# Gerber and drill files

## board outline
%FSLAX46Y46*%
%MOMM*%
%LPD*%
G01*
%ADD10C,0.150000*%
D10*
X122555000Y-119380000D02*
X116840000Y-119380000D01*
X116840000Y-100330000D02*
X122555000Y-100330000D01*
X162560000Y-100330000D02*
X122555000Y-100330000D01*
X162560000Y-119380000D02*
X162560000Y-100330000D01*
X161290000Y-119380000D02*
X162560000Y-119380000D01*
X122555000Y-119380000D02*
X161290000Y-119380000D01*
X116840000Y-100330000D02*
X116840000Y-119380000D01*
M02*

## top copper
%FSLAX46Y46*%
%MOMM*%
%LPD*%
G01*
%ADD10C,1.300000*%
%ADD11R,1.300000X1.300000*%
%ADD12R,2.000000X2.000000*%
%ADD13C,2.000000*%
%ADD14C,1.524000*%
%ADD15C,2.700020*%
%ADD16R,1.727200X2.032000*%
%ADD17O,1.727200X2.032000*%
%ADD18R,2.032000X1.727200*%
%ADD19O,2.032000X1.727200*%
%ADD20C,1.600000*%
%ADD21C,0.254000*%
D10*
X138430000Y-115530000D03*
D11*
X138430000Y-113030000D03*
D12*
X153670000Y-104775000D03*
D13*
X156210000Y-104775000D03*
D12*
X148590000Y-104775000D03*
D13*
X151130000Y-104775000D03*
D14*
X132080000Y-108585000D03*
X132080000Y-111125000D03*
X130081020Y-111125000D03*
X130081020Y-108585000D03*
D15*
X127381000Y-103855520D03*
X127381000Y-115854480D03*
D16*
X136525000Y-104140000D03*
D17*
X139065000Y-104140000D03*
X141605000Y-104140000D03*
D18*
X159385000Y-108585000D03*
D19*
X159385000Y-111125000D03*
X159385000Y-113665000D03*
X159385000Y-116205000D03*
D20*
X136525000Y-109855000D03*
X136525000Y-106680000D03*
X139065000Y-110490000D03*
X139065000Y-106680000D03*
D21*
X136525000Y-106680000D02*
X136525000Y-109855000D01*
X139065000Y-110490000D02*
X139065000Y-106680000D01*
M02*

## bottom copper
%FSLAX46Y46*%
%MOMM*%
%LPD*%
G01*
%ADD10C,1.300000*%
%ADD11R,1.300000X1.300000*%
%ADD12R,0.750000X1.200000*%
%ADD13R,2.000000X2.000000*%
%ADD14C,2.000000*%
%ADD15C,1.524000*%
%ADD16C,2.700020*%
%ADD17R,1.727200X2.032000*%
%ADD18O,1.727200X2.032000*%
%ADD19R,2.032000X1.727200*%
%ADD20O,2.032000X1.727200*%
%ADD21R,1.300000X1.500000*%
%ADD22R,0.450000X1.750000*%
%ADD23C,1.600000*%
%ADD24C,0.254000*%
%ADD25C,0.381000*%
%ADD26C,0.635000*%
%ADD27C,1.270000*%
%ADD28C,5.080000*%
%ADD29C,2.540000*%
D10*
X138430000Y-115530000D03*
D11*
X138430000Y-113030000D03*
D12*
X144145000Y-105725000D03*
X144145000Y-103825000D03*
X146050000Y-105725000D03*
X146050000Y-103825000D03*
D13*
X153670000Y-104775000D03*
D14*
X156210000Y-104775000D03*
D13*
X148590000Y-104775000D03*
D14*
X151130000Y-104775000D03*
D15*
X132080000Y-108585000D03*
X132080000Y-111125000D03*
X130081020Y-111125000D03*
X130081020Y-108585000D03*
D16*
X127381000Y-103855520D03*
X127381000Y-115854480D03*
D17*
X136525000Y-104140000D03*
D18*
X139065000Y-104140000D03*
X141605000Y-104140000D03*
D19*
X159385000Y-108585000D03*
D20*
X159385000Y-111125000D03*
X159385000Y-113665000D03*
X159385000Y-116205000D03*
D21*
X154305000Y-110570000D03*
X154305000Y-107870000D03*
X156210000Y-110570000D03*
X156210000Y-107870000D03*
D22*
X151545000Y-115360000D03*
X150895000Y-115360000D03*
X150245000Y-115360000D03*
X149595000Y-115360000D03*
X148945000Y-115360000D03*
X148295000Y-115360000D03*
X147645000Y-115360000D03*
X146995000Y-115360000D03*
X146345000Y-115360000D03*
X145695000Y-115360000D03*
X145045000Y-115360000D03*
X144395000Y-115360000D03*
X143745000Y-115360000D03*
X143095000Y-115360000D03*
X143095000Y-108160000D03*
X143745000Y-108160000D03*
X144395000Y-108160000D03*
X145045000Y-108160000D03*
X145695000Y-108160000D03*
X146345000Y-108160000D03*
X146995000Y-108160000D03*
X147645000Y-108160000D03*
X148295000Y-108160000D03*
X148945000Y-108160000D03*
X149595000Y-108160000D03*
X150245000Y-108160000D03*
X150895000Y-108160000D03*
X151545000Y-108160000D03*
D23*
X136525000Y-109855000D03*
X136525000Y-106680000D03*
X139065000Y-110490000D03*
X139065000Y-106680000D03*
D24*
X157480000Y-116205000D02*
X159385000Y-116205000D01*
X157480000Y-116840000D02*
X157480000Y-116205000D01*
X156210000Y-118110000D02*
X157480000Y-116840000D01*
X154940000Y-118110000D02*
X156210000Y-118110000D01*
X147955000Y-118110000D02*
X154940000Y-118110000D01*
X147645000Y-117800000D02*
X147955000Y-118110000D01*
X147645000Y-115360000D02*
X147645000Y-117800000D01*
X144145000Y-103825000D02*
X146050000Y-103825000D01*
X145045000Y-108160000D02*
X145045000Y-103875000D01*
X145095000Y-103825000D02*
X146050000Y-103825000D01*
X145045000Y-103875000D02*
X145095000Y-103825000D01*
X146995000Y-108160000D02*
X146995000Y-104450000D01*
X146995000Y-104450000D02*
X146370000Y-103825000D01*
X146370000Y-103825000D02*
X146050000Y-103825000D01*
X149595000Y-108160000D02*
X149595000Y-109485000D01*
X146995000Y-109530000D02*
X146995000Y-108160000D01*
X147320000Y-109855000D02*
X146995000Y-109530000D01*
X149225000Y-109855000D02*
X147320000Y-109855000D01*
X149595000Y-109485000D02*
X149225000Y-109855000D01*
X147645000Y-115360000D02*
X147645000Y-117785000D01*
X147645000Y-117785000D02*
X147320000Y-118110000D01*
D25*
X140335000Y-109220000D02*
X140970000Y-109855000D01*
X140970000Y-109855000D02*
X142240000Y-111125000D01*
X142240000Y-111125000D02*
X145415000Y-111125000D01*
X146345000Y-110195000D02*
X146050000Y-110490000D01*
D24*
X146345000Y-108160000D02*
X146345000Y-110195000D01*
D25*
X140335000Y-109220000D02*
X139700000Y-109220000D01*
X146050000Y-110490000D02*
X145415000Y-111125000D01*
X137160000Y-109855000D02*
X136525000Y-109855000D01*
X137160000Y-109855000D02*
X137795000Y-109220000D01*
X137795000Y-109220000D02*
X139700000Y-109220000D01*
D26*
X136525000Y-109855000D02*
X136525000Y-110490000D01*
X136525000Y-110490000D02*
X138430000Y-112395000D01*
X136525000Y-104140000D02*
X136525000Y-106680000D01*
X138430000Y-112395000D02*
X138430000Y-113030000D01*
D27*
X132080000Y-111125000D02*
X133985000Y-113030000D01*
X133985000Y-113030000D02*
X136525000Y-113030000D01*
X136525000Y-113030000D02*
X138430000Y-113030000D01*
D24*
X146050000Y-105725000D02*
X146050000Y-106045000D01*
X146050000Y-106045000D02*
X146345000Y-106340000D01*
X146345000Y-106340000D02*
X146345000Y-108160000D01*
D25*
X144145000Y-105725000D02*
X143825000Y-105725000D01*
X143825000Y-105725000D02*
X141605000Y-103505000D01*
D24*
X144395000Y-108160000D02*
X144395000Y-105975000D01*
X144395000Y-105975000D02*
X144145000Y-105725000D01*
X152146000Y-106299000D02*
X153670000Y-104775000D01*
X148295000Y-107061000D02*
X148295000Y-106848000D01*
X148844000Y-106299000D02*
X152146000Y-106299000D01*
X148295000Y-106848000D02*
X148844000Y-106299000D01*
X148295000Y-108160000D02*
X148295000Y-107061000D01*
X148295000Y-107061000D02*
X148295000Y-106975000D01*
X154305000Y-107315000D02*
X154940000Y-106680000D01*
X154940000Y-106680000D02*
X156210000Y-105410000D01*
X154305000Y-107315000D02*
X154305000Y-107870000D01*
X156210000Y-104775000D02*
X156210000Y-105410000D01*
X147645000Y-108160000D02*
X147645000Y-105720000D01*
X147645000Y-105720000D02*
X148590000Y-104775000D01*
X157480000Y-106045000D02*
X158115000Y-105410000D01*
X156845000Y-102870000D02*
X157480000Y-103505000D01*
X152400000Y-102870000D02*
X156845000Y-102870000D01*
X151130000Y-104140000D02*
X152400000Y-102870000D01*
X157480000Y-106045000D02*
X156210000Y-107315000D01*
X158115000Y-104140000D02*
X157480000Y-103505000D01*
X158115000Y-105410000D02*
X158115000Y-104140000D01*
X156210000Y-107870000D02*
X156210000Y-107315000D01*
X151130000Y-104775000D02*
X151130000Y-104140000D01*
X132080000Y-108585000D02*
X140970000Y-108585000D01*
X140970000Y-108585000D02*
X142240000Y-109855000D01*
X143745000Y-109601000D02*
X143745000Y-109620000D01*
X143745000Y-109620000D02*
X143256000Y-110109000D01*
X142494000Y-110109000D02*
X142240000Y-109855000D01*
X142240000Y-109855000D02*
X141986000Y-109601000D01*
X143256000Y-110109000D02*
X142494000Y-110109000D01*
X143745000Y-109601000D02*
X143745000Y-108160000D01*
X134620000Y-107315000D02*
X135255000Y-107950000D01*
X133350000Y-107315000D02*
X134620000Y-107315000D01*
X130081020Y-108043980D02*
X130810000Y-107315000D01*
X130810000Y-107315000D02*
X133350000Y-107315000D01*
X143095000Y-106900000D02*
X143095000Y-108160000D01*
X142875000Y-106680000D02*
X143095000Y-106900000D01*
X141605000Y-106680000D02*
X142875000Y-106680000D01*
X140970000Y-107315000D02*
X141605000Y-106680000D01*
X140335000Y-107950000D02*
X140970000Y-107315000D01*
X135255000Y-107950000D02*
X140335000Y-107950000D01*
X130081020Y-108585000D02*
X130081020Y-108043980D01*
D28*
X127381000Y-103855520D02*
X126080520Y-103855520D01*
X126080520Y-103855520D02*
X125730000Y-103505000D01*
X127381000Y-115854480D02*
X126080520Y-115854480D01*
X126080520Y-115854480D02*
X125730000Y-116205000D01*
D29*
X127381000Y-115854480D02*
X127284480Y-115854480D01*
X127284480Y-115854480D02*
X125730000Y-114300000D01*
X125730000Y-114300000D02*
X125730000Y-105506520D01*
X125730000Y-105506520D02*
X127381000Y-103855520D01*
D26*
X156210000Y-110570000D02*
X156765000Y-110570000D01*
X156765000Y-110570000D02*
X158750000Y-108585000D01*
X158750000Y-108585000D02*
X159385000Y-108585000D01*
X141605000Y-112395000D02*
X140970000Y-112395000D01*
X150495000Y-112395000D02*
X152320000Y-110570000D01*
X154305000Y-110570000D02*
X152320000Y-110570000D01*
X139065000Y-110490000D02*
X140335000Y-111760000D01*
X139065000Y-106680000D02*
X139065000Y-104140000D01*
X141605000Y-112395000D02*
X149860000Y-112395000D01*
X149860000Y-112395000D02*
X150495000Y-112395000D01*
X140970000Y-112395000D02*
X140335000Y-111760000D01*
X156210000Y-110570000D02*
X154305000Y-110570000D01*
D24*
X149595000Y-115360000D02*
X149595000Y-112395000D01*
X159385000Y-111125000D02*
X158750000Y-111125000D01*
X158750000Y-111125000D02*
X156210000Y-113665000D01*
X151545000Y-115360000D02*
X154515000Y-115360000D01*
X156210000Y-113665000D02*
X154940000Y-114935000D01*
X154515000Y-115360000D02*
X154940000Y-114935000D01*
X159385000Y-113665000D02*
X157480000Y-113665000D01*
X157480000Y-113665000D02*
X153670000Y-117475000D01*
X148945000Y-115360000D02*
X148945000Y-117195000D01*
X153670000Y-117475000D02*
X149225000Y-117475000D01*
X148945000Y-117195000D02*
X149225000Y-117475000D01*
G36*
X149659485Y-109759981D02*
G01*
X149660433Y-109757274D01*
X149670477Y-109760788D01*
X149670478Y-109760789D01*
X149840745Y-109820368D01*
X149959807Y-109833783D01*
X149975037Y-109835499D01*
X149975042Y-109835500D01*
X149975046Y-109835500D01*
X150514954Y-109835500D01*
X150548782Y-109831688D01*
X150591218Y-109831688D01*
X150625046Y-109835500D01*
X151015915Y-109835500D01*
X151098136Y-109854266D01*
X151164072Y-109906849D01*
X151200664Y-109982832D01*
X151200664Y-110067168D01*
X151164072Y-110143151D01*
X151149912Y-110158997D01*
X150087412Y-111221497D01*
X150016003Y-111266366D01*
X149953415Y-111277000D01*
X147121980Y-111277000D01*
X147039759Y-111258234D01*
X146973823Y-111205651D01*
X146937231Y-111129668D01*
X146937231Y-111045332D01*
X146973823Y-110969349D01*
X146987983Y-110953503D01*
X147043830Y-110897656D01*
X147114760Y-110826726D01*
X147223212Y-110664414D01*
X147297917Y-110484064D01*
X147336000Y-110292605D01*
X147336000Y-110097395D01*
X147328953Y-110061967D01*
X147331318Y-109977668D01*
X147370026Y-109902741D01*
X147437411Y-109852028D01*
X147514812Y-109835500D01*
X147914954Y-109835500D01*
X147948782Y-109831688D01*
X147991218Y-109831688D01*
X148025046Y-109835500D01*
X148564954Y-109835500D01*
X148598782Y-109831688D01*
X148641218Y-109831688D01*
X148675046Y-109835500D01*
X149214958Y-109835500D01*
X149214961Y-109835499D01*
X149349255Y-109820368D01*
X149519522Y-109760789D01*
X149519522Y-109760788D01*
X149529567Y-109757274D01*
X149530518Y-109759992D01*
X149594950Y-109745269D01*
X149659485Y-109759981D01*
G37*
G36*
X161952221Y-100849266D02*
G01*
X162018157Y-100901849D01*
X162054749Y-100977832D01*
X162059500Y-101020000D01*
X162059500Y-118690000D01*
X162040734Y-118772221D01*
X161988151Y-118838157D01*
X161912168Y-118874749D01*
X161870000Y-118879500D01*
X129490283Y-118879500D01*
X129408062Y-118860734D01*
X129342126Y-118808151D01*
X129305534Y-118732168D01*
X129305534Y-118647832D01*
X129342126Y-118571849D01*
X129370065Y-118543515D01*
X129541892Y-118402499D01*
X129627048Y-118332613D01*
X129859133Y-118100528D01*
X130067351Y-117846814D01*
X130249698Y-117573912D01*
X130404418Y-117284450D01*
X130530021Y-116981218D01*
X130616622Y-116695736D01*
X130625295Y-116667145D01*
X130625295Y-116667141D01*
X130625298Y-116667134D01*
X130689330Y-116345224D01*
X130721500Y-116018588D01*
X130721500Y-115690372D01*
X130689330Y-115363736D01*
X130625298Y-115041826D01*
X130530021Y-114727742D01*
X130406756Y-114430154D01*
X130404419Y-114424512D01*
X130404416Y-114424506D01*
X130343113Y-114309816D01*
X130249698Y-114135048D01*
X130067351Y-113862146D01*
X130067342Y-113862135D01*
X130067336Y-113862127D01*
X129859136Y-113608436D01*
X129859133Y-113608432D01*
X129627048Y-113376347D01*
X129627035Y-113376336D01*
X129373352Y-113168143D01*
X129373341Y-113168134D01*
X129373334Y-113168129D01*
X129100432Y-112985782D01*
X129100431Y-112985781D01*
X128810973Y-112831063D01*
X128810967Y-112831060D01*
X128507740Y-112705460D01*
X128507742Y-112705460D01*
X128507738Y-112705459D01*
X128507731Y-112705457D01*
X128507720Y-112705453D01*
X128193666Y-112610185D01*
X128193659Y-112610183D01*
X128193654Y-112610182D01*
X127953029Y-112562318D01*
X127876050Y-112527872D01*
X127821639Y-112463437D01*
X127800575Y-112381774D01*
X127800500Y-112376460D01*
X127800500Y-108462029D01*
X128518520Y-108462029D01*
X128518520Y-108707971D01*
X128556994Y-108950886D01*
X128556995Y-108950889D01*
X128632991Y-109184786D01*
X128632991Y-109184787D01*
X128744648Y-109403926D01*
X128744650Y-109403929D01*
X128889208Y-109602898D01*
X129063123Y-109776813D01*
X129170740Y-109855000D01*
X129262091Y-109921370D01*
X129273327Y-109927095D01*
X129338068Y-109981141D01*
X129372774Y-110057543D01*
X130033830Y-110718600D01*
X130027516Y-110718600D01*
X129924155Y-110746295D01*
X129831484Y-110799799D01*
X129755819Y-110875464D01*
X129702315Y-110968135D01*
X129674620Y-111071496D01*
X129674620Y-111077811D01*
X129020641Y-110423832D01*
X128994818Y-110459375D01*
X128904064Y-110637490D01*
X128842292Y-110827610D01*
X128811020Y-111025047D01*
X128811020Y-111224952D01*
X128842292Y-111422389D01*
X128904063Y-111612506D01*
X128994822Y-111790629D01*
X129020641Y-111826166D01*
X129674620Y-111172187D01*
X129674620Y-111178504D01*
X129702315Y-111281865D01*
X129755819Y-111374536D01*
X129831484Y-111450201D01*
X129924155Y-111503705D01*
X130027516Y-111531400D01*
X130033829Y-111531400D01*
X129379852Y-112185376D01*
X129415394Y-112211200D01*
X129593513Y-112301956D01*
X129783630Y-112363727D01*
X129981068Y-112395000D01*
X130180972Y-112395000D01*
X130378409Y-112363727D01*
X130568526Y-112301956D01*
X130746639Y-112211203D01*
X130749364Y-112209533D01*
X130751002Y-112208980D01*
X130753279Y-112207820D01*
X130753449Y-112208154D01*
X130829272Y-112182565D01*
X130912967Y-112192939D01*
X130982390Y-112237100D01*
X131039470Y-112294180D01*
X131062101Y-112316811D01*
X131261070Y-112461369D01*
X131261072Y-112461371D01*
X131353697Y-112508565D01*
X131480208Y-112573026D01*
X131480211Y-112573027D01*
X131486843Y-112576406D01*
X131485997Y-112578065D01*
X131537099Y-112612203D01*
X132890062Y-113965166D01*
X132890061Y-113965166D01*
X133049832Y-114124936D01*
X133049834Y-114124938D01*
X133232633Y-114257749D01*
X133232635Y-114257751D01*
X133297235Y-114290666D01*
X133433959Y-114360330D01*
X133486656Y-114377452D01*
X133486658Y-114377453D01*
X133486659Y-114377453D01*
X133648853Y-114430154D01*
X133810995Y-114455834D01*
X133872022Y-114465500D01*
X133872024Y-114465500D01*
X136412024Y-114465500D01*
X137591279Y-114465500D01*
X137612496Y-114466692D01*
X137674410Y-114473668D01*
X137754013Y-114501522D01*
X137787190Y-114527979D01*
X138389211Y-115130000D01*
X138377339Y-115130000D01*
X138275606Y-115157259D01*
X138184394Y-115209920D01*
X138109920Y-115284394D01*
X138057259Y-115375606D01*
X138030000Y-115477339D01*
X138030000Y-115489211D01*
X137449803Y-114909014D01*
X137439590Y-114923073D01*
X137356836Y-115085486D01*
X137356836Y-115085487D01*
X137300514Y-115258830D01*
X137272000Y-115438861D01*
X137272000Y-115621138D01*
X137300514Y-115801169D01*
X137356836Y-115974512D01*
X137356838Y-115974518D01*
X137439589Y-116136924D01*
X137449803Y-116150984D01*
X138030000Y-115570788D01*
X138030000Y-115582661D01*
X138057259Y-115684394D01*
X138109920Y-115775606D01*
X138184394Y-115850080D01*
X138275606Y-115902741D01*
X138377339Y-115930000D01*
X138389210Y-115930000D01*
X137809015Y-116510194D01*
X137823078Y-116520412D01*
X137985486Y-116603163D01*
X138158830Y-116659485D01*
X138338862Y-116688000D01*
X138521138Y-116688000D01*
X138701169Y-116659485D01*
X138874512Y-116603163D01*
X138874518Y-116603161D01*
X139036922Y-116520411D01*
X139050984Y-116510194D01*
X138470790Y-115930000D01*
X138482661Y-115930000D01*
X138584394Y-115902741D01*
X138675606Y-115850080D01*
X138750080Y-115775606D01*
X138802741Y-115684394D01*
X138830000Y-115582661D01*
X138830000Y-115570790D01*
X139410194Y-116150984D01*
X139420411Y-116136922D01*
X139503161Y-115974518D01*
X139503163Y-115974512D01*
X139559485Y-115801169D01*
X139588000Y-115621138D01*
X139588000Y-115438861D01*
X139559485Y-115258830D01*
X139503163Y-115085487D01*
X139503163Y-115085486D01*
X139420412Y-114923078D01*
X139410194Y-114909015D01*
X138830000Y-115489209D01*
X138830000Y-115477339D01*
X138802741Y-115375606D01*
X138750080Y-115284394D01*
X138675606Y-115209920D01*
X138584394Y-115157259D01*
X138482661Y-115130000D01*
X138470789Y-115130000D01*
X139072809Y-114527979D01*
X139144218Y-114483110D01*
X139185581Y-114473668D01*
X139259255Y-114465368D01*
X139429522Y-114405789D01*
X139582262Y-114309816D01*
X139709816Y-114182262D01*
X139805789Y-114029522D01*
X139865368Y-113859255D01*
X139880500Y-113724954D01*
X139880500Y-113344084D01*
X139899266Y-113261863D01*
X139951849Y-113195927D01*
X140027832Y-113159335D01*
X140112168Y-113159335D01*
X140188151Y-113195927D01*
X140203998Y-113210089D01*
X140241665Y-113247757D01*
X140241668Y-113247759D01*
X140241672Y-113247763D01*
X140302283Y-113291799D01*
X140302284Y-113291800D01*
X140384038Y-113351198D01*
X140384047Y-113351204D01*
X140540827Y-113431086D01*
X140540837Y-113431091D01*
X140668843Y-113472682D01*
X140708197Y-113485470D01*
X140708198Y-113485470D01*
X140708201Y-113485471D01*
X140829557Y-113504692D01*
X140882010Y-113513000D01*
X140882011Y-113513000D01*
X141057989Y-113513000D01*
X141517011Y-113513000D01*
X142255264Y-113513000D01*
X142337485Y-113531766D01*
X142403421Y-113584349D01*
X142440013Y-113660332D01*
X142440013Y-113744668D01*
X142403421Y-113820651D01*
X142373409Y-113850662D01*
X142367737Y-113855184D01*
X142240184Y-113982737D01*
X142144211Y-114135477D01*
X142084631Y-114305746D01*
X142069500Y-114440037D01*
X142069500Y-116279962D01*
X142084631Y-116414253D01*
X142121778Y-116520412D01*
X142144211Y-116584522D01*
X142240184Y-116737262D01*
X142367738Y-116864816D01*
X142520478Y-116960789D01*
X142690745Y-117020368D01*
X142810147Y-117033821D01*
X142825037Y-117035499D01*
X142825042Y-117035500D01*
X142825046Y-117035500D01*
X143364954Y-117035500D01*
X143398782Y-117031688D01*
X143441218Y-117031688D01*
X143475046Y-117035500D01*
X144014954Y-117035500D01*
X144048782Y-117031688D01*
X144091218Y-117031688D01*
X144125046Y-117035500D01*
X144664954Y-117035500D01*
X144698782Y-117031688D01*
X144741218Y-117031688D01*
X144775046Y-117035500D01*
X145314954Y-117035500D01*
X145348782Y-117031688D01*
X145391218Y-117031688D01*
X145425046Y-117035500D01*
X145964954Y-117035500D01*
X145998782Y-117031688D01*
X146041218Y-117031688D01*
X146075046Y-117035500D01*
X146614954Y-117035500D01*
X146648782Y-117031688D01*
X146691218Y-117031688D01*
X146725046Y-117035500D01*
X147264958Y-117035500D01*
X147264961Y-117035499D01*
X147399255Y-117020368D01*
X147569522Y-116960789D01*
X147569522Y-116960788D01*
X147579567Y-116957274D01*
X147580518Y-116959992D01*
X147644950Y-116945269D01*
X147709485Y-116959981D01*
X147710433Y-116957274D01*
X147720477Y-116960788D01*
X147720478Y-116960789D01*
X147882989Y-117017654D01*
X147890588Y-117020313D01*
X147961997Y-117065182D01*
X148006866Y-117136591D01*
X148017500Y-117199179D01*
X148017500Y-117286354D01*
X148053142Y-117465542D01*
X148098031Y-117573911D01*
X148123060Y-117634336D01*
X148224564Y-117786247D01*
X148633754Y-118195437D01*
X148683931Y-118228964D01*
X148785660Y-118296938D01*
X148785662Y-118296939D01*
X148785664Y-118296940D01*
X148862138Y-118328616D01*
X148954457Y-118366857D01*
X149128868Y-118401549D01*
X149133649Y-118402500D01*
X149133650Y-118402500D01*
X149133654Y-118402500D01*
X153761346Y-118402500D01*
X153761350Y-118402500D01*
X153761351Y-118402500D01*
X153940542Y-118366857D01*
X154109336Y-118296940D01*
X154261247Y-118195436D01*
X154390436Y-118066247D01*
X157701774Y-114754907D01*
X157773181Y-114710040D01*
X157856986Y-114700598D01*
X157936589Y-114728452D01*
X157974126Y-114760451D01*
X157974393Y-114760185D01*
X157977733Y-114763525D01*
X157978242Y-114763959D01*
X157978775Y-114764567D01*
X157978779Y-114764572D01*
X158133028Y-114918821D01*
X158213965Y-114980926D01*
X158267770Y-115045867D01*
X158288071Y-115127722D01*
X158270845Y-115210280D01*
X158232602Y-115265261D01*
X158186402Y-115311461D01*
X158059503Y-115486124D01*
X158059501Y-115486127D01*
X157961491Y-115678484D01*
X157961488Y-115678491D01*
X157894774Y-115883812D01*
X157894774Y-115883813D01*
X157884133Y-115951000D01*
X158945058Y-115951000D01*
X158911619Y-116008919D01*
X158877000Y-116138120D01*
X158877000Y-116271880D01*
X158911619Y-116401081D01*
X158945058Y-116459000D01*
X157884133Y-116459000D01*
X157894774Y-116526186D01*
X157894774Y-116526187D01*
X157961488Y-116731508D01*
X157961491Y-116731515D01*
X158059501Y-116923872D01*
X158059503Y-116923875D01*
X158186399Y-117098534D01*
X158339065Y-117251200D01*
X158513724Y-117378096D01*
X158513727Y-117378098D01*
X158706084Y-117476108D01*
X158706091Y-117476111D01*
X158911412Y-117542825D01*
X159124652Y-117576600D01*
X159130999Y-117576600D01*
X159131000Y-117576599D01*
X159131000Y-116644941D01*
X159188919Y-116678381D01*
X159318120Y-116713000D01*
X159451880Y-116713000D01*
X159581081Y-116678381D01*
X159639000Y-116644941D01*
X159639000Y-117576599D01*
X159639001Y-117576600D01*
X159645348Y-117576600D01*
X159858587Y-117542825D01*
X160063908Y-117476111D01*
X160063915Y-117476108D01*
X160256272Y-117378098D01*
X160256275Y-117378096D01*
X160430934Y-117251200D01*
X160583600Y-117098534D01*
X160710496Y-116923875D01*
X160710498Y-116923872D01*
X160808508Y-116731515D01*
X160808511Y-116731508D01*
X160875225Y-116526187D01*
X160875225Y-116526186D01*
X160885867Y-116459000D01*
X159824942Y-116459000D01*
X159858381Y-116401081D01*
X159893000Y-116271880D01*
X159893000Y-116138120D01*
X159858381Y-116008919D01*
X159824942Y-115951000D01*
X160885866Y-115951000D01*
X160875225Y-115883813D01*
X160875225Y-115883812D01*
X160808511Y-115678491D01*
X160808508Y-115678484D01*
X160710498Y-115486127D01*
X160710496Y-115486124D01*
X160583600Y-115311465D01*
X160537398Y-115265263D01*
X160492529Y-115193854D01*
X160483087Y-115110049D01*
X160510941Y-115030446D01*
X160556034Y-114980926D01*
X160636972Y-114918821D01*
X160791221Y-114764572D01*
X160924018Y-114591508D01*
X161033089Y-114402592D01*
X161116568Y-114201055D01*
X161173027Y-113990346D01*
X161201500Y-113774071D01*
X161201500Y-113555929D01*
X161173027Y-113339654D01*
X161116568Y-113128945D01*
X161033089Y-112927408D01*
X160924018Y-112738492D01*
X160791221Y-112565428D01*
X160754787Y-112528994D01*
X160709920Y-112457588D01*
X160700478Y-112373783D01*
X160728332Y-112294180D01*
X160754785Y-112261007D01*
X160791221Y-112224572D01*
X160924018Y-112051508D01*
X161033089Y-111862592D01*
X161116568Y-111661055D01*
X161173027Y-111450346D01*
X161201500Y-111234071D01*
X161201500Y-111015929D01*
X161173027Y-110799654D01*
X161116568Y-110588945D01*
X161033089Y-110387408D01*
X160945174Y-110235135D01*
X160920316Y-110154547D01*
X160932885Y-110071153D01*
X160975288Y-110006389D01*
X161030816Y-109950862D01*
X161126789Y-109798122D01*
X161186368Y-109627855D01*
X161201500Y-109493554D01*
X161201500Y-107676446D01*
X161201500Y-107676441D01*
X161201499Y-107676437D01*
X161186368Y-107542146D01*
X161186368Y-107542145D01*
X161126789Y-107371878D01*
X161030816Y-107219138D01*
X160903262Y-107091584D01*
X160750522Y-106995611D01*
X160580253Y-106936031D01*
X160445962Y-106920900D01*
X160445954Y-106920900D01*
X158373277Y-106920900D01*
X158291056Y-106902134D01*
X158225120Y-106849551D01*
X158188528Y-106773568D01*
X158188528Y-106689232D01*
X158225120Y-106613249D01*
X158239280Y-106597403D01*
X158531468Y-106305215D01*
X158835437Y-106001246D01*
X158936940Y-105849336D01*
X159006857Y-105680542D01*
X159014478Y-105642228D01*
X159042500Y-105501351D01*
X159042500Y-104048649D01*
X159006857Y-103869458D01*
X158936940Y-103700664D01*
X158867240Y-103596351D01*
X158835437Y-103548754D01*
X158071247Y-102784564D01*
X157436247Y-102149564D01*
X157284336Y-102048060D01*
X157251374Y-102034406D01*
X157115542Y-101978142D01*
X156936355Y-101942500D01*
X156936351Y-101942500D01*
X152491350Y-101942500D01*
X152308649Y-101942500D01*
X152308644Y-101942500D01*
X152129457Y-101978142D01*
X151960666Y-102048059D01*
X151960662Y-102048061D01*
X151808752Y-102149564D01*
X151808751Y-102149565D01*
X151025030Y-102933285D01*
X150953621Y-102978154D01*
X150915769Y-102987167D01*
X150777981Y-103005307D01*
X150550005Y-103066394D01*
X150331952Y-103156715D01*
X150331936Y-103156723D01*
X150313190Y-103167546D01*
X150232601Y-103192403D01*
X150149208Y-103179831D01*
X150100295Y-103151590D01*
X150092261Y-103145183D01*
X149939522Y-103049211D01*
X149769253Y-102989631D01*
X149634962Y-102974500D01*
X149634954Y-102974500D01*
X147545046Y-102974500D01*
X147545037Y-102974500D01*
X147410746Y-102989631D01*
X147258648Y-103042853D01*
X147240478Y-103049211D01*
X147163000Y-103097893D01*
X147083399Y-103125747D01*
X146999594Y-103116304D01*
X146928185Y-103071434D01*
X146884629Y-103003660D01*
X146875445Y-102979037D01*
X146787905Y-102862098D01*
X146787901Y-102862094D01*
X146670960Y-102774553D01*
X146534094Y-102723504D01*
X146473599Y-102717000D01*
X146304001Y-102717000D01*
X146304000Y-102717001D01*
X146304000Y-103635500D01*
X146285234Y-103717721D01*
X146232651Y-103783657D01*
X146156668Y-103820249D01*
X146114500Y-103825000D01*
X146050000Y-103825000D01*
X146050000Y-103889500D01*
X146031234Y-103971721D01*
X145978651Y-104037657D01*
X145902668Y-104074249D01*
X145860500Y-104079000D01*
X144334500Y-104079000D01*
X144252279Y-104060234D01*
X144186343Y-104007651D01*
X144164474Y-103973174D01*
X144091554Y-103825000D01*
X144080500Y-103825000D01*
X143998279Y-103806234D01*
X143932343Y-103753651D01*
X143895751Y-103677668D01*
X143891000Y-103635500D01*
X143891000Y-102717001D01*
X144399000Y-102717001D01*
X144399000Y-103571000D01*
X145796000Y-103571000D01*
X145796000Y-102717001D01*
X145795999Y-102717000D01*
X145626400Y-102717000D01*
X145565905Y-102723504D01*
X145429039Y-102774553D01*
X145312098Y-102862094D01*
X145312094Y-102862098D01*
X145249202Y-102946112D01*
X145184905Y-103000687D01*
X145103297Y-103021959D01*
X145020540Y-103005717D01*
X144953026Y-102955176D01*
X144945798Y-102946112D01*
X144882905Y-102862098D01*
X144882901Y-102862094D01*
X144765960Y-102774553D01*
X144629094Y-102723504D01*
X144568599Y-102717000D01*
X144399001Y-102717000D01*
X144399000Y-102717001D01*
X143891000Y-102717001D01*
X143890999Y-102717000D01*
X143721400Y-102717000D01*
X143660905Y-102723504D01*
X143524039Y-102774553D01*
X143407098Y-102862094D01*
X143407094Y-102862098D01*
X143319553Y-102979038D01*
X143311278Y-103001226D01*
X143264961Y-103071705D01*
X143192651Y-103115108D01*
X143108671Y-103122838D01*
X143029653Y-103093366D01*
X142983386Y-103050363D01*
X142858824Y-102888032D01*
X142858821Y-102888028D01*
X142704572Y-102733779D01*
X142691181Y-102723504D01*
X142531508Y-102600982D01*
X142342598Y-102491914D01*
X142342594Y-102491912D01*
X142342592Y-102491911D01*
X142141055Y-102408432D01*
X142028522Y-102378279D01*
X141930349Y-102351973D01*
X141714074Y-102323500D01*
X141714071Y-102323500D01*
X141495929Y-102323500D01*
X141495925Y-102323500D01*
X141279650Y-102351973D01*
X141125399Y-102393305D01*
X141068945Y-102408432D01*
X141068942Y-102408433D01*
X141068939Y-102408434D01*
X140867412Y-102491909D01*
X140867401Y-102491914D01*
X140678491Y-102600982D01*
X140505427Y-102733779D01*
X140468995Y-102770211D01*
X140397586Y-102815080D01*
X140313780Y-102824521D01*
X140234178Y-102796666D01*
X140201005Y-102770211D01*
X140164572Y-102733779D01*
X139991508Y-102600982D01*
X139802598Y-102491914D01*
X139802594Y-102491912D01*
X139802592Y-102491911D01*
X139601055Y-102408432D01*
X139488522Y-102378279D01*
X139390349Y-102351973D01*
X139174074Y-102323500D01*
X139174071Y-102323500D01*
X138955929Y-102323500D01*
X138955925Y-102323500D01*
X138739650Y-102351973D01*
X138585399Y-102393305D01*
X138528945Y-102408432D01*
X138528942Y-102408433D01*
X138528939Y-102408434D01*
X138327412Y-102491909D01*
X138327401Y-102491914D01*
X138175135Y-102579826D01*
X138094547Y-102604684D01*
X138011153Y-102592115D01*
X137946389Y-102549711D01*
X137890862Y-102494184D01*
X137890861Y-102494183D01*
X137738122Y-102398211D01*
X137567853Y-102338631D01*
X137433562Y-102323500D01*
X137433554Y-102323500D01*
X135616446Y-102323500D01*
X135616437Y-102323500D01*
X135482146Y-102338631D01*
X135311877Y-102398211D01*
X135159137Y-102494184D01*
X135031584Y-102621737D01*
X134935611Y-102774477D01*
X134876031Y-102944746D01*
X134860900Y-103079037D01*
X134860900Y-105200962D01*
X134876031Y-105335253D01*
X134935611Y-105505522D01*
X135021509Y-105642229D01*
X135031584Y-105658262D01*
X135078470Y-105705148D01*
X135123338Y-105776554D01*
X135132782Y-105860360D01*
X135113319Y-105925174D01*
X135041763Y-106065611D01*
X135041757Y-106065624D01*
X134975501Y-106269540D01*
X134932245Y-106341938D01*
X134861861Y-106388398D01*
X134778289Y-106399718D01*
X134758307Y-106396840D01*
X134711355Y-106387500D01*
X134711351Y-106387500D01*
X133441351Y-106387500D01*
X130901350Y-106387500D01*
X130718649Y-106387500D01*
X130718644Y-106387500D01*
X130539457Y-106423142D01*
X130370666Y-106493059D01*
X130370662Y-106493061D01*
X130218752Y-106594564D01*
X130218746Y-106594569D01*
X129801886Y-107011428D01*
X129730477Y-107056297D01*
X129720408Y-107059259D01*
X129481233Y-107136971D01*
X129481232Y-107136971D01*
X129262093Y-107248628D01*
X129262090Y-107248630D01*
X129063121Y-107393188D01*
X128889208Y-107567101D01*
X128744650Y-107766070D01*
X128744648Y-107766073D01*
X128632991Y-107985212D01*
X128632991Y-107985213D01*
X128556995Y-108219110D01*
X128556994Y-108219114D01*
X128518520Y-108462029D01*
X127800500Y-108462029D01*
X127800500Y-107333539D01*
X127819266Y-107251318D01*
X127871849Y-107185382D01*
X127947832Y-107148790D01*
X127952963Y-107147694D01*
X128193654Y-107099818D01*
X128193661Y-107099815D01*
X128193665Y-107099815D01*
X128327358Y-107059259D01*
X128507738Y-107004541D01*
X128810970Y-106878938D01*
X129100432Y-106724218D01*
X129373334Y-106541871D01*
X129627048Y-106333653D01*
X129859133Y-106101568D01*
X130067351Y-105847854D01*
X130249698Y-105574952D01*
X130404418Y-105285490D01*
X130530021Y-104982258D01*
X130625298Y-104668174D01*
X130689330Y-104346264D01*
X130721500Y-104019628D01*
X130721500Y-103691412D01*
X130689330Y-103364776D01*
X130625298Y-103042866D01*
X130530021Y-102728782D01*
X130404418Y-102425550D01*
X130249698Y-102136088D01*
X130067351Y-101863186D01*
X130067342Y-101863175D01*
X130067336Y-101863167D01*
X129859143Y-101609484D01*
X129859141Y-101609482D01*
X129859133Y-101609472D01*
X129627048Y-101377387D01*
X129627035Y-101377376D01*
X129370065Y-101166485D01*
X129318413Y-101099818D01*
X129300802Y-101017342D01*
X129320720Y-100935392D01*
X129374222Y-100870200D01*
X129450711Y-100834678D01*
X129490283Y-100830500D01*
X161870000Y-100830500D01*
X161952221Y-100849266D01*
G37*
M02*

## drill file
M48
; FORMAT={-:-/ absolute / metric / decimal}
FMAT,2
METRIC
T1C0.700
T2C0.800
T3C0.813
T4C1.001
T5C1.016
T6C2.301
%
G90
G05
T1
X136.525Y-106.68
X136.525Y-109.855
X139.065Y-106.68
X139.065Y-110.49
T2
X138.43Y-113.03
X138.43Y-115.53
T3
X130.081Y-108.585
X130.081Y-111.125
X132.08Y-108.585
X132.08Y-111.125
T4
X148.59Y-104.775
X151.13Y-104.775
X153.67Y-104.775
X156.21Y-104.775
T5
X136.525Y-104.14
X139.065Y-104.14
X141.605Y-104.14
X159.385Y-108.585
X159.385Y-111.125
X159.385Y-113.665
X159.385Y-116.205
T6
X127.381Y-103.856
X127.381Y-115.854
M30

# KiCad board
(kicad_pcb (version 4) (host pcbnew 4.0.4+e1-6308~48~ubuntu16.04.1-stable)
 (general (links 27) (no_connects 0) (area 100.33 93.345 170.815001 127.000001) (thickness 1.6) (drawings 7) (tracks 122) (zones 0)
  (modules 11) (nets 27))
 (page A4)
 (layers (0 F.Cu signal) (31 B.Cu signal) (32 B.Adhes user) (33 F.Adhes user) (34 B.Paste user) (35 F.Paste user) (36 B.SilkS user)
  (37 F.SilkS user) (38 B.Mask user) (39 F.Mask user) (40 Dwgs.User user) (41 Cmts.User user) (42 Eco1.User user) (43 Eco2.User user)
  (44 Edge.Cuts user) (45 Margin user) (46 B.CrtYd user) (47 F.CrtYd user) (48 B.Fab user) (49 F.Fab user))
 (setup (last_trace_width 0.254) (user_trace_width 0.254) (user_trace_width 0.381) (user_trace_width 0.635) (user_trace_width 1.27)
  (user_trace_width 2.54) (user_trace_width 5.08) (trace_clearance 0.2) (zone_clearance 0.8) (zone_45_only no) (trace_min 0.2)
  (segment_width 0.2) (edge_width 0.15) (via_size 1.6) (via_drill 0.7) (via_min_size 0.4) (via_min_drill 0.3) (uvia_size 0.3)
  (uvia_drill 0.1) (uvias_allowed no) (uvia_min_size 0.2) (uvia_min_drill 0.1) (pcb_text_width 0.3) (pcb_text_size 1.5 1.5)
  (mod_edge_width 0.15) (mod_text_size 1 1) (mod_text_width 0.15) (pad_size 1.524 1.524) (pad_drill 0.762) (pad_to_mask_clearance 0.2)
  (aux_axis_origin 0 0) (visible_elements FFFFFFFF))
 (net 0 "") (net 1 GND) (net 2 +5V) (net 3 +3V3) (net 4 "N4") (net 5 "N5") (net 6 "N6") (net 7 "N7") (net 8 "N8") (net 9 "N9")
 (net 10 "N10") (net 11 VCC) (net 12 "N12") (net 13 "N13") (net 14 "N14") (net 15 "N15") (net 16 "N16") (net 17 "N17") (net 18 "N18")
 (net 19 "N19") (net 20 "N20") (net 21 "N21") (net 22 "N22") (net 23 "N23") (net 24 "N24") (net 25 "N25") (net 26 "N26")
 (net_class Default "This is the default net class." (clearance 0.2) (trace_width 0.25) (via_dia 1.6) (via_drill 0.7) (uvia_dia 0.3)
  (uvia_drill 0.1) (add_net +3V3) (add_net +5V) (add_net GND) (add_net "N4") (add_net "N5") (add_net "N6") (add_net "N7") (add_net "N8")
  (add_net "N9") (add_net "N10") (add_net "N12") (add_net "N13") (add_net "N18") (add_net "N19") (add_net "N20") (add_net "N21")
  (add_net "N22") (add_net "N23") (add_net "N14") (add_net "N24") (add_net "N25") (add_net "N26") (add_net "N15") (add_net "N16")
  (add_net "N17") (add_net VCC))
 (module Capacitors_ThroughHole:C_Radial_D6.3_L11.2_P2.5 (layer F.Cu) (at 138.43 113.03 270)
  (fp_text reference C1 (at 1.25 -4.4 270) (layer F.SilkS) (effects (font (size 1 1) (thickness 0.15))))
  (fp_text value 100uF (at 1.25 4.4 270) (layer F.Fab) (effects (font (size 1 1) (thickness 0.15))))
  (pad 2 thru_hole circle (at 2.5 0 270) (size 1.3 1.3) (drill 0.8) (layers *.Cu *.Mask F.SilkS) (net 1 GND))
  (pad 1 thru_hole rect (at 0 0 270) (size 1.3 1.3) (drill 0.8) (layers *.Cu *.Mask F.SilkS) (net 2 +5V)))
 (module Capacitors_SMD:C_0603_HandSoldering (layer B.Cu) (at 144.145 104.775 90)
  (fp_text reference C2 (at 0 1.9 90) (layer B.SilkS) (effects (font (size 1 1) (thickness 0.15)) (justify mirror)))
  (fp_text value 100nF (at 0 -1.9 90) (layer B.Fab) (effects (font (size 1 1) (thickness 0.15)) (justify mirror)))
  (pad 1 smd rect (at -0.95 0 90) (size 1.2 0.75) (layers B.Cu B.Paste B.Mask) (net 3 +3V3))
  (pad 2 smd rect (at 0.95 0 90) (size 1.2 0.75) (layers B.Cu B.Paste B.Mask) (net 1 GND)))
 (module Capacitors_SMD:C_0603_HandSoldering (layer B.Cu) (at 146.05 104.775 90)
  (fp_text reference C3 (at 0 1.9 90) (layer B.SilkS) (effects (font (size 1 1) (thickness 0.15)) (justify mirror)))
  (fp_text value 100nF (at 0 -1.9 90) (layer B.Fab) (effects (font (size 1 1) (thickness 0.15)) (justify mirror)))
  (pad 1 smd rect (at -0.95 0 90) (size 1.2 0.75) (layers B.Cu B.Paste B.Mask) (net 2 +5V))
  (pad 2 smd rect (at 0.95 0 90) (size 1.2 0.75) (layers B.Cu B.Paste B.Mask) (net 1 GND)))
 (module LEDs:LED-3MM (layer F.Cu) (at 153.67 104.775)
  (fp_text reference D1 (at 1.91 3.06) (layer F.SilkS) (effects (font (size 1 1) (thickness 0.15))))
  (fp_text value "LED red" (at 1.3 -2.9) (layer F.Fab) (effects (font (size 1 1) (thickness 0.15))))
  (pad 1 thru_hole rect (at 0 0 90) (size 2 2) (drill 1.00076) (layers *.Cu *.Mask F.SilkS) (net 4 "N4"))
  (pad 2 thru_hole circle (at 2.54 0) (size 2 2) (drill 1.00076) (layers *.Cu *.Mask F.SilkS) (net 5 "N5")))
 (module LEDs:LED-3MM (layer F.Cu) (at 148.59 104.775)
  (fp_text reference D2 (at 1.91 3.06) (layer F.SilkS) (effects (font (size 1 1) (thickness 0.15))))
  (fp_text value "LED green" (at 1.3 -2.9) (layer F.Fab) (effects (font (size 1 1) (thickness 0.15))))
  (pad 1 thru_hole rect (at 0 0 90) (size 2 2) (drill 1.00076) (layers *.Cu *.Mask F.SilkS) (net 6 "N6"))
  (pad 2 thru_hole circle (at 2.54 0) (size 2 2) (drill 1.00076) (layers *.Cu *.Mask F.SilkS) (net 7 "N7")))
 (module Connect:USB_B (layer F.Cu) (at 132.08 111.125 180)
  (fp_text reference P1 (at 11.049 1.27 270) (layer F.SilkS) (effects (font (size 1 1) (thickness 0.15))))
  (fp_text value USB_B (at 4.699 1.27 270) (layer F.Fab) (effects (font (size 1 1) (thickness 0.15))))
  (pad 2 thru_hole circle (at 0 2.54 90) (size 1.524 1.524) (drill 0.8128) (layers *.Cu *.Mask F.SilkS) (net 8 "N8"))
  (pad 1 thru_hole circle (at 0 0 90) (size 1.524 1.524) (drill 0.8128) (layers *.Cu *.Mask F.SilkS) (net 2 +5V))
  (pad 4 thru_hole circle (at 1.99898 0 90) (size 1.524 1.524) (drill 0.8128) (layers *.Cu *.Mask F.SilkS) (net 1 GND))
  (pad 3 thru_hole circle (at 1.99898 2.54 90) (size 1.524 1.524) (drill 0.8128) (layers *.Cu *.Mask F.SilkS) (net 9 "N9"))
  (pad 5 thru_hole circle (at 4.699 7.26948 90) (size 2.70002 2.70002) (drill 2.30124) (layers *.Cu *.Mask F.SilkS) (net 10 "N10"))
  (pad 5 thru_hole circle (at 4.699 -4.72948 90) (size 2.70002 2.70002) (drill 2.30124) (layers *.Cu *.Mask F.SilkS) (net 10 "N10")))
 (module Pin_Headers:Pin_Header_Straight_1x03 (layer F.Cu) (at 136.525 104.14 90)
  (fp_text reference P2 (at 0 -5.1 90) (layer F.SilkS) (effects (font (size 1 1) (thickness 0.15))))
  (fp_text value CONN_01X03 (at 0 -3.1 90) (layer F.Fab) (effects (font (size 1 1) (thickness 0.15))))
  (pad 1 thru_hole rect (at 0 0 90) (size 2.032 1.7272) (drill 1.016) (layers *.Cu *.Mask F.SilkS) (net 2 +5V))
  (pad 2 thru_hole oval (at 0 2.54 90) (size 2.032 1.7272) (drill 1.016) (layers *.Cu *.Mask F.SilkS) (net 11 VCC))
  (pad 3 thru_hole oval (at 0 5.08 90) (size 2.032 1.7272) (drill 1.016) (layers *.Cu *.Mask F.SilkS) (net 3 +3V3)))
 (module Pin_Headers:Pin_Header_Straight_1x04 (layer F.Cu) (at 159.385 108.585)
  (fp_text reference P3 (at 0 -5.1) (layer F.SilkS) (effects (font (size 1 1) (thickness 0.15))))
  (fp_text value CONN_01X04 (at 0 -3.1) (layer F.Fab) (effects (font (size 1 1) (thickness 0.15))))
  (pad 1 thru_hole rect (at 0 0) (size 2.032 1.7272) (drill 1.016) (layers *.Cu *.Mask F.SilkS) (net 11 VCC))
  (pad 2 thru_hole oval (at 0 2.54) (size 2.032 1.7272) (drill 1.016) (layers *.Cu *.Mask F.SilkS) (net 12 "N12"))
  (pad 3 thru_hole oval (at 0 5.08) (size 2.032 1.7272) (drill 1.016) (layers *.Cu *.Mask F.SilkS) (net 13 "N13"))
  (pad 4 thru_hole oval (at 0 7.62) (size 2.032 1.7272) (drill 1.016) (layers *.Cu *.Mask F.SilkS) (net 1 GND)))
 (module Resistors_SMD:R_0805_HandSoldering (layer B.Cu) (at 154.305 109.22 90)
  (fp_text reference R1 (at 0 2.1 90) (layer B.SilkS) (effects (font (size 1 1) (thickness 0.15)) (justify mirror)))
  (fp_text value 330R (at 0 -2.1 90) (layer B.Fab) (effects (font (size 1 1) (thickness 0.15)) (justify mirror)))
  (pad 1 smd rect (at -1.35 0 90) (size 1.5 1.3) (layers B.Cu B.Paste B.Mask) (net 11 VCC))
  (pad 2 smd rect (at 1.35 0 90) (size 1.5 1.3) (layers B.Cu B.Paste B.Mask) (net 5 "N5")))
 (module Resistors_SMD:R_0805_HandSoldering (layer B.Cu) (at 156.21 109.22 90)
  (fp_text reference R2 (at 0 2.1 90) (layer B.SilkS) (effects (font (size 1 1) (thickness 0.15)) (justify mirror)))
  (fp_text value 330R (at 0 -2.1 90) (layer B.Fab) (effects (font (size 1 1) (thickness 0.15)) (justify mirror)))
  (pad 1 smd rect (at -1.35 0 90) (size 1.5 1.3) (layers B.Cu B.Paste B.Mask) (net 11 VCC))
  (pad 2 smd rect (at 1.35 0 90) (size 1.5 1.3) (layers B.Cu B.Paste B.Mask) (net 7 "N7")))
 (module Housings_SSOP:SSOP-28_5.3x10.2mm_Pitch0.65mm (layer B.Cu) (at 147.32 111.76 90)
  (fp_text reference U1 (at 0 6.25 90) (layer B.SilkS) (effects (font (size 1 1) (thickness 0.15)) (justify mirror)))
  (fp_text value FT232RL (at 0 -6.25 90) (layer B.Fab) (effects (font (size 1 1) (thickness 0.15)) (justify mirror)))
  (pad 1 smd rect (at -3.6 4.225 90) (size 1.75 0.45) (layers B.Cu B.Paste B.Mask) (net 12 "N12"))
  (pad 2 smd rect (at -3.6 3.575 90) (size 1.75 0.45) (layers B.Cu B.Paste B.Mask) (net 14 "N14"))
  (pad 3 smd rect (at -3.6 2.925 90) (size 1.75 0.45) (layers B.Cu B.Paste B.Mask) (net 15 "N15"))
  (pad 4 smd rect (at -3.6 2.275 90) (size 1.75 0.45) (layers B.Cu B.Paste B.Mask) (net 11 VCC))
  (pad 5 smd rect (at -3.6 1.625 90) (size 1.75 0.45) (layers B.Cu B.Paste B.Mask) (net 13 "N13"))
  (pad 6 smd rect (at -3.6 0.975 90) (size 1.75 0.45) (layers B.Cu B.Paste B.Mask) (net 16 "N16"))
  (pad 7 smd rect (at -3.6 0.325 90) (size 1.75 0.45) (layers B.Cu B.Paste B.Mask) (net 1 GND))
  (pad 8 smd rect (at -3.6 -0.325 90) (size 1.75 0.45) (layers B.Cu B.Paste B.Mask))
  (pad 9 smd rect (at -3.6 -0.975 90) (size 1.75 0.45) (layers B.Cu B.Paste B.Mask) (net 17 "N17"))
  (pad 10 smd rect (at -3.6 -1.625 90) (size 1.75 0.45) (layers B.Cu B.Paste B.Mask) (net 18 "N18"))
  (pad 11 smd rect (at -3.6 -2.275 90) (size 1.75 0.45) (layers B.Cu B.Paste B.Mask) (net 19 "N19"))
  (pad 12 smd rect (at -3.6 -2.925 90) (size 1.75 0.45) (layers B.Cu B.Paste B.Mask) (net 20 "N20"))
  (pad 13 smd rect (at -3.6 -3.575 90) (size 1.75 0.45) (layers B.Cu B.Paste B.Mask) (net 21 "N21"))
  (pad 14 smd rect (at -3.6 -4.225 90) (size 1.75 0.45) (layers B.Cu B.Paste B.Mask) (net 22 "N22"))
  (pad 15 smd rect (at 3.6 -4.225 90) (size 1.75 0.45) (layers B.Cu B.Paste B.Mask) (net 9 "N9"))
  (pad 16 smd rect (at 3.6 -3.575 90) (size 1.75 0.45) (layers B.Cu B.Paste B.Mask) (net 8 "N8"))
  (pad 17 smd rect (at 3.6 -2.925 90) (size 1.75 0.45) (layers B.Cu B.Paste B.Mask) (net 3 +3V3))
  (pad 18 smd rect (at 3.6 -2.275 90) (size 1.75 0.45) (layers B.Cu B.Paste B.Mask) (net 1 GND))
  (pad 19 smd rect (at 3.6 -1.625 90) (size 1.75 0.45) (layers B.Cu B.Paste B.Mask) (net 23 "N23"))
  (pad 20 smd rect (at 3.6 -0.975 90) (size 1.75 0.45) (layers B.Cu B.Paste B.Mask) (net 2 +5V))
  (pad 21 smd rect (at 3.6 -0.325 90) (size 1.75 0.45) (layers B.Cu B.Paste B.Mask) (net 1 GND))
  (pad 22 smd rect (at 3.6 0.325 90) (size 1.75 0.45) (layers B.Cu B.Paste B.Mask) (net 6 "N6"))
  (pad 23 smd rect (at 3.6 0.975 90) (size 1.75 0.45) (layers B.Cu B.Paste B.Mask) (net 4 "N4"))
  (pad 24 smd rect (at 3.6 1.625 90) (size 1.75 0.45) (layers B.Cu B.Paste B.Mask))
  (pad 25 smd rect (at 3.6 2.275 90) (size 1.75 0.45) (layers B.Cu B.Paste B.Mask) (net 1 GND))
  (pad 26 smd rect (at 3.6 2.925 90) (size 1.75 0.45) (layers B.Cu B.Paste B.Mask) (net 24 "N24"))
  (pad 27 smd rect (at 3.6 3.575 90) (size 1.75 0.45) (layers B.Cu B.Paste B.Mask) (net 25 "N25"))
  (pad 28 smd rect (at 3.6 4.225 90) (size 1.75 0.45) (layers B.Cu B.Paste B.Mask) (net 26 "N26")))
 (gr_line (start 122.555 119.38) (end 116.84 119.38) (angle 90) (layer Edge.Cuts) (width 0.15))
 (gr_line (start 116.84 100.33) (end 122.555 100.33) (angle 90) (layer Edge.Cuts) (width 0.15))
 (gr_line (start 162.56 100.33) (end 122.555 100.33) (angle 90) (layer Edge.Cuts) (width 0.15))
 (gr_line (start 162.56 119.38) (end 162.56 100.33) (angle 90) (layer Edge.Cuts) (width 0.15))
 (gr_line (start 161.29 119.38) (end 162.56 119.38) (angle 90) (layer Edge.Cuts) (width 0.15))
 (gr_line (start 122.555 119.38) (end 161.29 119.38) (angle 90) (layer Edge.Cuts) (width 0.15))
 (gr_line (start 116.84 100.33) (end 116.84 119.38) (angle 90) (layer Edge.Cuts) (width 0.15))
 (segment (start 157.48 116.205) (end 159.385 116.205) (width 0.254) (layer B.Cu) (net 1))
 (segment (start 157.48 116.84) (end 157.48 116.205) (width 0.254) (layer B.Cu) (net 1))
 (segment (start 156.21 118.11) (end 157.48 116.84) (width 0.254) (layer B.Cu) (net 1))
 (segment (start 154.94 118.11) (end 156.21 118.11) (width 0.254) (layer B.Cu) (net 1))
 (segment (start 147.955 118.11) (end 154.94 118.11) (width 0.254) (layer B.Cu) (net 1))
 (segment (start 147.645 117.8) (end 147.955 118.11) (width 0.254) (layer B.Cu) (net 1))
 (segment (start 147.645 115.36) (end 147.645 117.8) (width 0.254) (layer B.Cu) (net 1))
 (segment (start 144.145 103.825) (end 146.05 103.825) (width 0.254) (layer B.Cu) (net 1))
 (segment (start 145.045 108.16) (end 145.045 103.875) (width 0.254) (layer B.Cu) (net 1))
 (segment (start 145.095 103.825) (end 146.05 103.825) (width 0.254) (layer B.Cu) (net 1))
 (segment (start 145.045 103.875) (end 145.095 103.825) (width 0.254) (layer B.Cu) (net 1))
 (segment (start 146.995 108.16) (end 146.995 104.45) (width 0.254) (layer B.Cu) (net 1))
 (segment (start 146.995 104.45) (end 146.37 103.825) (width 0.254) (layer B.Cu) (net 1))
 (segment (start 146.37 103.825) (end 146.05 103.825) (width 0.254) (layer B.Cu) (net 1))
 (segment (start 149.595 108.16) (end 149.595 109.485) (width 0.254) (layer B.Cu) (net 1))
 (segment (start 146.995 109.53) (end 146.995 108.16) (width 0.254) (layer B.Cu) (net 1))
 (segment (start 147.32 109.855) (end 146.995 109.53) (width 0.254) (layer B.Cu) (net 1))
 (segment (start 149.225 109.855) (end 147.32 109.855) (width 0.254) (layer B.Cu) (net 1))
 (segment (start 149.595 109.485) (end 149.225 109.855) (width 0.254) (layer B.Cu) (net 1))
 (segment (start 147.645 115.36) (end 147.645 117.785) (width 0.254) (layer B.Cu) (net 1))
 (segment (start 147.645 117.785) (end 147.32 118.11) (width 0.254) (layer B.Cu) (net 1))
 (segment (start 140.335 109.22) (end 140.97 109.855) (width 0.381) (layer B.Cu) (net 2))
 (segment (start 140.97 109.855) (end 142.24 111.125) (width 0.381) (layer B.Cu) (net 2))
 (segment (start 142.24 111.125) (end 145.415 111.125) (width 0.381) (layer B.Cu) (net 2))
 (segment (start 146.345 110.195) (end 146.05 110.49) (width 0.381) (layer B.Cu) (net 2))
 (segment (start 146.345 108.16) (end 146.345 110.195) (width 0.254) (layer B.Cu) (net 2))
 (segment (start 140.335 109.22) (end 139.7 109.22) (width 0.381) (layer B.Cu) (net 2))
 (segment (start 146.05 110.49) (end 145.415 111.125) (width 0.381) (layer B.Cu) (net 2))
 (segment (start 137.16 109.855) (end 136.525 109.855) (width 0.381) (layer B.Cu) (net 2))
 (segment (start 137.16 109.855) (end 137.795 109.22) (width 0.381) (layer B.Cu) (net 2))
 (segment (start 137.795 109.22) (end 139.7 109.22) (width 0.381) (layer B.Cu) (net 2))
 (segment (start 136.525 109.855) (end 136.525 110.49) (width 0.635) (layer B.Cu) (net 2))
 (segment (start 136.525 110.49) (end 138.43 112.395) (width 0.635) (layer B.Cu) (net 2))
 (via (at 136.525 109.855) (size 1.6) (drill 0.7) (layers F.Cu B.Cu) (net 2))
 (segment (start 136.525 106.68) (end 136.525 109.855) (width 0.254) (layer F.Cu) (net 2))
 (via (at 136.525 106.68) (size 1.6) (drill 0.7) (layers F.Cu B.Cu) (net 2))
 (segment (start 136.525 104.14) (end 136.525 106.68) (width 0.635) (layer B.Cu) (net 2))
 (segment (start 138.43 112.395) (end 138.43 113.03) (width 0.635) (layer B.Cu) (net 2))
 (segment (start 132.08 111.125) (end 133.985 113.03) (width 1.27) (layer B.Cu) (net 2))
 (segment (start 133.985 113.03) (end 136.525 113.03) (width 1.27) (layer B.Cu) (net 2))
 (segment (start 136.525 113.03) (end 138.43 113.03) (width 1.27) (layer B.Cu) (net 2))
 (segment (start 146.05 105.725) (end 146.05 106.045) (width 0.254) (layer B.Cu) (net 2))
 (segment (start 146.05 106.045) (end 146.345 106.34) (width 0.254) (layer B.Cu) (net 2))
 (segment (start 146.345 106.34) (end 146.345 108.16) (width 0.254) (layer B.Cu) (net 2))
 (segment (start 144.145 105.725) (end 143.825 105.725) (width 0.381) (layer B.Cu) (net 3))
 (segment (start 143.825 105.725) (end 141.605 103.505) (width 0.381) (layer B.Cu) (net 3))
 (segment (start 144.395 108.16) (end 144.395 105.975) (width 0.254) (layer B.Cu) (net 3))
 (segment (start 144.395 105.975) (end 144.145 105.725) (width 0.254) (layer B.Cu) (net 3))
 (segment (start 152.146 106.299) (end 153.67 104.775) (width 0.254) (layer B.Cu) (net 4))
 (segment (start 148.295 107.061) (end 148.295 106.848) (width 0.254) (layer B.Cu) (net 4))
 (segment (start 148.844 106.299) (end 152.146 106.299) (width 0.254) (layer B.Cu) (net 4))
 (segment (start 148.295 106.848) (end 148.844 106.299) (width 0.254) (layer B.Cu) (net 4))
 (segment (start 148.295 108.16) (end 148.295 107.061) (width 0.254) (layer B.Cu) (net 4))
 (segment (start 148.295 107.061) (end 148.295 106.975) (width 0.254) (layer B.Cu) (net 4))
 (segment (start 154.305 107.315) (end 154.94 106.68) (width 0.254) (layer B.Cu) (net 5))
 (segment (start 154.94 106.68) (end 156.21 105.41) (width 0.254) (layer B.Cu) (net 5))
 (segment (start 154.305 107.315) (end 154.305 107.87) (width 0.254) (layer B.Cu) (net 5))
 (segment (start 156.21 104.775) (end 156.21 105.41) (width 0.254) (layer B.Cu) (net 5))
 (segment (start 147.645 108.16) (end 147.645 105.72) (width 0.254) (layer B.Cu) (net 6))
 (segment (start 147.645 105.72) (end 148.59 104.775) (width 0.254) (layer B.Cu) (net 6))
 (segment (start 157.48 106.045) (end 158.115 105.41) (width 0.254) (layer B.Cu) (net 7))
 (segment (start 156.845 102.87) (end 157.48 103.505) (width 0.254) (layer B.Cu) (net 7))
 (segment (start 152.4 102.87) (end 156.845 102.87) (width 0.254) (layer B.Cu) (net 7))
 (segment (start 151.13 104.14) (end 152.4 102.87) (width 0.254) (layer B.Cu) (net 7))
 (segment (start 157.48 106.045) (end 156.21 107.315) (width 0.254) (layer B.Cu) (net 7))
 (segment (start 158.115 104.14) (end 157.48 103.505) (width 0.254) (layer B.Cu) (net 7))
 (segment (start 158.115 105.41) (end 158.115 104.14) (width 0.254) (layer B.Cu) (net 7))
 (segment (start 156.21 107.87) (end 156.21 107.315) (width 0.254) (layer B.Cu) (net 7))
 (segment (start 151.13 104.775) (end 151.13 104.14) (width 0.254) (layer B.Cu) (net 7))
 (segment (start 132.08 108.585) (end 140.97 108.585) (width 0.254) (layer B.Cu) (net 8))
 (segment (start 140.97 108.585) (end 142.24 109.855) (width 0.254) (layer B.Cu) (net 8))
 (segment (start 143.745 109.601) (end 143.745 109.62) (width 0.254) (layer B.Cu) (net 8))
 (segment (start 143.745 109.62) (end 143.256 110.109) (width 0.254) (layer B.Cu) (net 8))
 (segment (start 142.494 110.109) (end 142.24 109.855) (width 0.254) (layer B.Cu) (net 8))
 (segment (start 142.24 109.855) (end 141.986 109.601) (width 0.254) (layer B.Cu) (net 8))
 (segment (start 143.256 110.109) (end 142.494 110.109) (width 0.254) (layer B.Cu) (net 8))
 (segment (start 143.745 109.601) (end 143.745 108.16) (width 0.254) (layer B.Cu) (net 8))
 (segment (start 134.62 107.315) (end 135.255 107.95) (width 0.254) (layer B.Cu) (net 9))
 (segment (start 133.35 107.315) (end 134.62 107.315) (width 0.254) (layer B.Cu) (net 9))
 (segment (start 130.08102 108.04398) (end 130.81 107.315) (width 0.254) (layer B.Cu) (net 9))
 (segment (start 130.81 107.315) (end 133.35 107.315) (width 0.254) (layer B.Cu) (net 9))
 (segment (start 143.095 106.9) (end 143.095 108.16) (width 0.254) (layer B.Cu) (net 9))
 (segment (start 142.875 106.68) (end 143.095 106.9) (width 0.254) (layer B.Cu) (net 9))
 (segment (start 141.605 106.68) (end 142.875 106.68) (width 0.254) (layer B.Cu) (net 9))
 (segment (start 140.97 107.315) (end 141.605 106.68) (width 0.254) (layer B.Cu) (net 9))
 (segment (start 140.335 107.95) (end 140.97 107.315) (width 0.254) (layer B.Cu) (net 9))
 (segment (start 135.255 107.95) (end 140.335 107.95) (width 0.254) (layer B.Cu) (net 9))
 (segment (start 130.08102 108.585) (end 130.08102 108.04398) (width 0.254) (layer B.Cu) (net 9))
 (segment (start 127.381 103.85552) (end 126.08052 103.85552) (width 5.08) (layer B.Cu) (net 10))
 (segment (start 126.08052 103.85552) (end 125.73 103.505) (width 5.08) (layer B.Cu) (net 10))
 (segment (start 127.381 115.85448) (end 126.08052 115.85448) (width 5.08) (layer B.Cu) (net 10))
 (segment (start 126.08052 115.85448) (end 125.73 116.205) (width 5.08) (layer B.Cu) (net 10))
 (segment (start 127.381 115.85448) (end 127.28448 115.85448) (width 2.54) (layer B.Cu) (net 10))
 (segment (start 127.28448 115.85448) (end 125.73 114.3) (width 2.54) (layer B.Cu) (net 10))
 (segment (start 125.73 114.3) (end 125.73 105.50652) (width 2.54) (layer B.Cu) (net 10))
 (segment (start 125.73 105.50652) (end 127.381 103.85552) (width 2.54) (layer B.Cu) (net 10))
 (segment (start 156.21 110.57) (end 156.765 110.57) (width 0.635) (layer B.Cu) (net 11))
 (segment (start 156.765 110.57) (end 158.75 108.585) (width 0.635) (layer B.Cu) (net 11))
 (segment (start 158.75 108.585) (end 159.385 108.585) (width 0.635) (layer B.Cu) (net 11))
 (segment (start 141.605 112.395) (end 140.97 112.395) (width 0.635) (layer B.Cu) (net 11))
 (segment (start 150.495 112.395) (end 152.32 110.57) (width 0.635) (layer B.Cu) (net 11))
 (segment (start 154.305 110.57) (end 152.32 110.57) (width 0.635) (layer B.Cu) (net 11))
 (segment (start 139.065 110.49) (end 140.335 111.76) (width 0.635) (layer B.Cu) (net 11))
 (via (at 139.065 110.49) (size 1.6) (drill 0.7) (layers F.Cu B.Cu) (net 11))
 (segment (start 139.065 106.68) (end 139.065 104.14) (width 0.635) (layer B.Cu) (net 11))
 (via (at 139.065 106.68) (size 1.6) (drill 0.7) (layers F.Cu B.Cu) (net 11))
 (segment (start 139.065 110.49) (end 139.065 106.68) (width 0.254) (layer F.Cu) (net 11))
 (segment (start 141.605 112.395) (end 149.86 112.395) (width 0.635) (layer B.Cu) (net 11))
 (segment (start 149.86 112.395) (end 150.495 112.395) (width 0.635) (layer B.Cu) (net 11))
 (segment (start 140.97 112.395) (end 140.335 111.76) (width 0.635) (layer B.Cu) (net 11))
 (segment (start 156.21 110.57) (end 154.305 110.57) (width 0.635) (layer B.Cu) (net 11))
 (segment (start 149.595 115.36) (end 149.595 112.395) (width 0.254) (layer B.Cu) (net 11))
 (segment (start 159.385 111.125) (end 158.75 111.125) (width 0.254) (layer B.Cu) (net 12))
 (segment (start 158.75 111.125) (end 156.21 113.665) (width 0.254) (layer B.Cu) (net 12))
 (segment (start 151.545 115.36) (end 154.515 115.36) (width 0.254) (layer B.Cu) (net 12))
 (segment (start 156.21 113.665) (end 154.94 114.935) (width 0.254) (layer B.Cu) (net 12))
 (segment (start 154.515 115.36) (end 154.94 114.935) (width 0.254) (layer B.Cu) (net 12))
 (segment (start 159.385 113.665) (end 157.48 113.665) (width 0.254) (layer B.Cu) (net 13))
 (segment (start 157.48 113.665) (end 153.67 117.475) (width 0.254) (layer B.Cu) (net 13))
 (segment (start 148.945 115.36) (end 148.945 117.195) (width 0.254) (layer B.Cu) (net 13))
 (segment (start 153.67 117.475) (end 149.225 117.475) (width 0.254) (layer B.Cu) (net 13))
 (segment (start 148.945 117.195) (end 149.225 117.475) (width 0.254) (layer B.Cu) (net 13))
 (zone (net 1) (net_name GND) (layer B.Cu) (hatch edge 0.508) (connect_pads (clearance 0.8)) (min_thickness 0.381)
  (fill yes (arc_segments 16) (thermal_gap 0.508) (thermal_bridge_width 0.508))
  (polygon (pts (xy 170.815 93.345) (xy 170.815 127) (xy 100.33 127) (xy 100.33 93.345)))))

